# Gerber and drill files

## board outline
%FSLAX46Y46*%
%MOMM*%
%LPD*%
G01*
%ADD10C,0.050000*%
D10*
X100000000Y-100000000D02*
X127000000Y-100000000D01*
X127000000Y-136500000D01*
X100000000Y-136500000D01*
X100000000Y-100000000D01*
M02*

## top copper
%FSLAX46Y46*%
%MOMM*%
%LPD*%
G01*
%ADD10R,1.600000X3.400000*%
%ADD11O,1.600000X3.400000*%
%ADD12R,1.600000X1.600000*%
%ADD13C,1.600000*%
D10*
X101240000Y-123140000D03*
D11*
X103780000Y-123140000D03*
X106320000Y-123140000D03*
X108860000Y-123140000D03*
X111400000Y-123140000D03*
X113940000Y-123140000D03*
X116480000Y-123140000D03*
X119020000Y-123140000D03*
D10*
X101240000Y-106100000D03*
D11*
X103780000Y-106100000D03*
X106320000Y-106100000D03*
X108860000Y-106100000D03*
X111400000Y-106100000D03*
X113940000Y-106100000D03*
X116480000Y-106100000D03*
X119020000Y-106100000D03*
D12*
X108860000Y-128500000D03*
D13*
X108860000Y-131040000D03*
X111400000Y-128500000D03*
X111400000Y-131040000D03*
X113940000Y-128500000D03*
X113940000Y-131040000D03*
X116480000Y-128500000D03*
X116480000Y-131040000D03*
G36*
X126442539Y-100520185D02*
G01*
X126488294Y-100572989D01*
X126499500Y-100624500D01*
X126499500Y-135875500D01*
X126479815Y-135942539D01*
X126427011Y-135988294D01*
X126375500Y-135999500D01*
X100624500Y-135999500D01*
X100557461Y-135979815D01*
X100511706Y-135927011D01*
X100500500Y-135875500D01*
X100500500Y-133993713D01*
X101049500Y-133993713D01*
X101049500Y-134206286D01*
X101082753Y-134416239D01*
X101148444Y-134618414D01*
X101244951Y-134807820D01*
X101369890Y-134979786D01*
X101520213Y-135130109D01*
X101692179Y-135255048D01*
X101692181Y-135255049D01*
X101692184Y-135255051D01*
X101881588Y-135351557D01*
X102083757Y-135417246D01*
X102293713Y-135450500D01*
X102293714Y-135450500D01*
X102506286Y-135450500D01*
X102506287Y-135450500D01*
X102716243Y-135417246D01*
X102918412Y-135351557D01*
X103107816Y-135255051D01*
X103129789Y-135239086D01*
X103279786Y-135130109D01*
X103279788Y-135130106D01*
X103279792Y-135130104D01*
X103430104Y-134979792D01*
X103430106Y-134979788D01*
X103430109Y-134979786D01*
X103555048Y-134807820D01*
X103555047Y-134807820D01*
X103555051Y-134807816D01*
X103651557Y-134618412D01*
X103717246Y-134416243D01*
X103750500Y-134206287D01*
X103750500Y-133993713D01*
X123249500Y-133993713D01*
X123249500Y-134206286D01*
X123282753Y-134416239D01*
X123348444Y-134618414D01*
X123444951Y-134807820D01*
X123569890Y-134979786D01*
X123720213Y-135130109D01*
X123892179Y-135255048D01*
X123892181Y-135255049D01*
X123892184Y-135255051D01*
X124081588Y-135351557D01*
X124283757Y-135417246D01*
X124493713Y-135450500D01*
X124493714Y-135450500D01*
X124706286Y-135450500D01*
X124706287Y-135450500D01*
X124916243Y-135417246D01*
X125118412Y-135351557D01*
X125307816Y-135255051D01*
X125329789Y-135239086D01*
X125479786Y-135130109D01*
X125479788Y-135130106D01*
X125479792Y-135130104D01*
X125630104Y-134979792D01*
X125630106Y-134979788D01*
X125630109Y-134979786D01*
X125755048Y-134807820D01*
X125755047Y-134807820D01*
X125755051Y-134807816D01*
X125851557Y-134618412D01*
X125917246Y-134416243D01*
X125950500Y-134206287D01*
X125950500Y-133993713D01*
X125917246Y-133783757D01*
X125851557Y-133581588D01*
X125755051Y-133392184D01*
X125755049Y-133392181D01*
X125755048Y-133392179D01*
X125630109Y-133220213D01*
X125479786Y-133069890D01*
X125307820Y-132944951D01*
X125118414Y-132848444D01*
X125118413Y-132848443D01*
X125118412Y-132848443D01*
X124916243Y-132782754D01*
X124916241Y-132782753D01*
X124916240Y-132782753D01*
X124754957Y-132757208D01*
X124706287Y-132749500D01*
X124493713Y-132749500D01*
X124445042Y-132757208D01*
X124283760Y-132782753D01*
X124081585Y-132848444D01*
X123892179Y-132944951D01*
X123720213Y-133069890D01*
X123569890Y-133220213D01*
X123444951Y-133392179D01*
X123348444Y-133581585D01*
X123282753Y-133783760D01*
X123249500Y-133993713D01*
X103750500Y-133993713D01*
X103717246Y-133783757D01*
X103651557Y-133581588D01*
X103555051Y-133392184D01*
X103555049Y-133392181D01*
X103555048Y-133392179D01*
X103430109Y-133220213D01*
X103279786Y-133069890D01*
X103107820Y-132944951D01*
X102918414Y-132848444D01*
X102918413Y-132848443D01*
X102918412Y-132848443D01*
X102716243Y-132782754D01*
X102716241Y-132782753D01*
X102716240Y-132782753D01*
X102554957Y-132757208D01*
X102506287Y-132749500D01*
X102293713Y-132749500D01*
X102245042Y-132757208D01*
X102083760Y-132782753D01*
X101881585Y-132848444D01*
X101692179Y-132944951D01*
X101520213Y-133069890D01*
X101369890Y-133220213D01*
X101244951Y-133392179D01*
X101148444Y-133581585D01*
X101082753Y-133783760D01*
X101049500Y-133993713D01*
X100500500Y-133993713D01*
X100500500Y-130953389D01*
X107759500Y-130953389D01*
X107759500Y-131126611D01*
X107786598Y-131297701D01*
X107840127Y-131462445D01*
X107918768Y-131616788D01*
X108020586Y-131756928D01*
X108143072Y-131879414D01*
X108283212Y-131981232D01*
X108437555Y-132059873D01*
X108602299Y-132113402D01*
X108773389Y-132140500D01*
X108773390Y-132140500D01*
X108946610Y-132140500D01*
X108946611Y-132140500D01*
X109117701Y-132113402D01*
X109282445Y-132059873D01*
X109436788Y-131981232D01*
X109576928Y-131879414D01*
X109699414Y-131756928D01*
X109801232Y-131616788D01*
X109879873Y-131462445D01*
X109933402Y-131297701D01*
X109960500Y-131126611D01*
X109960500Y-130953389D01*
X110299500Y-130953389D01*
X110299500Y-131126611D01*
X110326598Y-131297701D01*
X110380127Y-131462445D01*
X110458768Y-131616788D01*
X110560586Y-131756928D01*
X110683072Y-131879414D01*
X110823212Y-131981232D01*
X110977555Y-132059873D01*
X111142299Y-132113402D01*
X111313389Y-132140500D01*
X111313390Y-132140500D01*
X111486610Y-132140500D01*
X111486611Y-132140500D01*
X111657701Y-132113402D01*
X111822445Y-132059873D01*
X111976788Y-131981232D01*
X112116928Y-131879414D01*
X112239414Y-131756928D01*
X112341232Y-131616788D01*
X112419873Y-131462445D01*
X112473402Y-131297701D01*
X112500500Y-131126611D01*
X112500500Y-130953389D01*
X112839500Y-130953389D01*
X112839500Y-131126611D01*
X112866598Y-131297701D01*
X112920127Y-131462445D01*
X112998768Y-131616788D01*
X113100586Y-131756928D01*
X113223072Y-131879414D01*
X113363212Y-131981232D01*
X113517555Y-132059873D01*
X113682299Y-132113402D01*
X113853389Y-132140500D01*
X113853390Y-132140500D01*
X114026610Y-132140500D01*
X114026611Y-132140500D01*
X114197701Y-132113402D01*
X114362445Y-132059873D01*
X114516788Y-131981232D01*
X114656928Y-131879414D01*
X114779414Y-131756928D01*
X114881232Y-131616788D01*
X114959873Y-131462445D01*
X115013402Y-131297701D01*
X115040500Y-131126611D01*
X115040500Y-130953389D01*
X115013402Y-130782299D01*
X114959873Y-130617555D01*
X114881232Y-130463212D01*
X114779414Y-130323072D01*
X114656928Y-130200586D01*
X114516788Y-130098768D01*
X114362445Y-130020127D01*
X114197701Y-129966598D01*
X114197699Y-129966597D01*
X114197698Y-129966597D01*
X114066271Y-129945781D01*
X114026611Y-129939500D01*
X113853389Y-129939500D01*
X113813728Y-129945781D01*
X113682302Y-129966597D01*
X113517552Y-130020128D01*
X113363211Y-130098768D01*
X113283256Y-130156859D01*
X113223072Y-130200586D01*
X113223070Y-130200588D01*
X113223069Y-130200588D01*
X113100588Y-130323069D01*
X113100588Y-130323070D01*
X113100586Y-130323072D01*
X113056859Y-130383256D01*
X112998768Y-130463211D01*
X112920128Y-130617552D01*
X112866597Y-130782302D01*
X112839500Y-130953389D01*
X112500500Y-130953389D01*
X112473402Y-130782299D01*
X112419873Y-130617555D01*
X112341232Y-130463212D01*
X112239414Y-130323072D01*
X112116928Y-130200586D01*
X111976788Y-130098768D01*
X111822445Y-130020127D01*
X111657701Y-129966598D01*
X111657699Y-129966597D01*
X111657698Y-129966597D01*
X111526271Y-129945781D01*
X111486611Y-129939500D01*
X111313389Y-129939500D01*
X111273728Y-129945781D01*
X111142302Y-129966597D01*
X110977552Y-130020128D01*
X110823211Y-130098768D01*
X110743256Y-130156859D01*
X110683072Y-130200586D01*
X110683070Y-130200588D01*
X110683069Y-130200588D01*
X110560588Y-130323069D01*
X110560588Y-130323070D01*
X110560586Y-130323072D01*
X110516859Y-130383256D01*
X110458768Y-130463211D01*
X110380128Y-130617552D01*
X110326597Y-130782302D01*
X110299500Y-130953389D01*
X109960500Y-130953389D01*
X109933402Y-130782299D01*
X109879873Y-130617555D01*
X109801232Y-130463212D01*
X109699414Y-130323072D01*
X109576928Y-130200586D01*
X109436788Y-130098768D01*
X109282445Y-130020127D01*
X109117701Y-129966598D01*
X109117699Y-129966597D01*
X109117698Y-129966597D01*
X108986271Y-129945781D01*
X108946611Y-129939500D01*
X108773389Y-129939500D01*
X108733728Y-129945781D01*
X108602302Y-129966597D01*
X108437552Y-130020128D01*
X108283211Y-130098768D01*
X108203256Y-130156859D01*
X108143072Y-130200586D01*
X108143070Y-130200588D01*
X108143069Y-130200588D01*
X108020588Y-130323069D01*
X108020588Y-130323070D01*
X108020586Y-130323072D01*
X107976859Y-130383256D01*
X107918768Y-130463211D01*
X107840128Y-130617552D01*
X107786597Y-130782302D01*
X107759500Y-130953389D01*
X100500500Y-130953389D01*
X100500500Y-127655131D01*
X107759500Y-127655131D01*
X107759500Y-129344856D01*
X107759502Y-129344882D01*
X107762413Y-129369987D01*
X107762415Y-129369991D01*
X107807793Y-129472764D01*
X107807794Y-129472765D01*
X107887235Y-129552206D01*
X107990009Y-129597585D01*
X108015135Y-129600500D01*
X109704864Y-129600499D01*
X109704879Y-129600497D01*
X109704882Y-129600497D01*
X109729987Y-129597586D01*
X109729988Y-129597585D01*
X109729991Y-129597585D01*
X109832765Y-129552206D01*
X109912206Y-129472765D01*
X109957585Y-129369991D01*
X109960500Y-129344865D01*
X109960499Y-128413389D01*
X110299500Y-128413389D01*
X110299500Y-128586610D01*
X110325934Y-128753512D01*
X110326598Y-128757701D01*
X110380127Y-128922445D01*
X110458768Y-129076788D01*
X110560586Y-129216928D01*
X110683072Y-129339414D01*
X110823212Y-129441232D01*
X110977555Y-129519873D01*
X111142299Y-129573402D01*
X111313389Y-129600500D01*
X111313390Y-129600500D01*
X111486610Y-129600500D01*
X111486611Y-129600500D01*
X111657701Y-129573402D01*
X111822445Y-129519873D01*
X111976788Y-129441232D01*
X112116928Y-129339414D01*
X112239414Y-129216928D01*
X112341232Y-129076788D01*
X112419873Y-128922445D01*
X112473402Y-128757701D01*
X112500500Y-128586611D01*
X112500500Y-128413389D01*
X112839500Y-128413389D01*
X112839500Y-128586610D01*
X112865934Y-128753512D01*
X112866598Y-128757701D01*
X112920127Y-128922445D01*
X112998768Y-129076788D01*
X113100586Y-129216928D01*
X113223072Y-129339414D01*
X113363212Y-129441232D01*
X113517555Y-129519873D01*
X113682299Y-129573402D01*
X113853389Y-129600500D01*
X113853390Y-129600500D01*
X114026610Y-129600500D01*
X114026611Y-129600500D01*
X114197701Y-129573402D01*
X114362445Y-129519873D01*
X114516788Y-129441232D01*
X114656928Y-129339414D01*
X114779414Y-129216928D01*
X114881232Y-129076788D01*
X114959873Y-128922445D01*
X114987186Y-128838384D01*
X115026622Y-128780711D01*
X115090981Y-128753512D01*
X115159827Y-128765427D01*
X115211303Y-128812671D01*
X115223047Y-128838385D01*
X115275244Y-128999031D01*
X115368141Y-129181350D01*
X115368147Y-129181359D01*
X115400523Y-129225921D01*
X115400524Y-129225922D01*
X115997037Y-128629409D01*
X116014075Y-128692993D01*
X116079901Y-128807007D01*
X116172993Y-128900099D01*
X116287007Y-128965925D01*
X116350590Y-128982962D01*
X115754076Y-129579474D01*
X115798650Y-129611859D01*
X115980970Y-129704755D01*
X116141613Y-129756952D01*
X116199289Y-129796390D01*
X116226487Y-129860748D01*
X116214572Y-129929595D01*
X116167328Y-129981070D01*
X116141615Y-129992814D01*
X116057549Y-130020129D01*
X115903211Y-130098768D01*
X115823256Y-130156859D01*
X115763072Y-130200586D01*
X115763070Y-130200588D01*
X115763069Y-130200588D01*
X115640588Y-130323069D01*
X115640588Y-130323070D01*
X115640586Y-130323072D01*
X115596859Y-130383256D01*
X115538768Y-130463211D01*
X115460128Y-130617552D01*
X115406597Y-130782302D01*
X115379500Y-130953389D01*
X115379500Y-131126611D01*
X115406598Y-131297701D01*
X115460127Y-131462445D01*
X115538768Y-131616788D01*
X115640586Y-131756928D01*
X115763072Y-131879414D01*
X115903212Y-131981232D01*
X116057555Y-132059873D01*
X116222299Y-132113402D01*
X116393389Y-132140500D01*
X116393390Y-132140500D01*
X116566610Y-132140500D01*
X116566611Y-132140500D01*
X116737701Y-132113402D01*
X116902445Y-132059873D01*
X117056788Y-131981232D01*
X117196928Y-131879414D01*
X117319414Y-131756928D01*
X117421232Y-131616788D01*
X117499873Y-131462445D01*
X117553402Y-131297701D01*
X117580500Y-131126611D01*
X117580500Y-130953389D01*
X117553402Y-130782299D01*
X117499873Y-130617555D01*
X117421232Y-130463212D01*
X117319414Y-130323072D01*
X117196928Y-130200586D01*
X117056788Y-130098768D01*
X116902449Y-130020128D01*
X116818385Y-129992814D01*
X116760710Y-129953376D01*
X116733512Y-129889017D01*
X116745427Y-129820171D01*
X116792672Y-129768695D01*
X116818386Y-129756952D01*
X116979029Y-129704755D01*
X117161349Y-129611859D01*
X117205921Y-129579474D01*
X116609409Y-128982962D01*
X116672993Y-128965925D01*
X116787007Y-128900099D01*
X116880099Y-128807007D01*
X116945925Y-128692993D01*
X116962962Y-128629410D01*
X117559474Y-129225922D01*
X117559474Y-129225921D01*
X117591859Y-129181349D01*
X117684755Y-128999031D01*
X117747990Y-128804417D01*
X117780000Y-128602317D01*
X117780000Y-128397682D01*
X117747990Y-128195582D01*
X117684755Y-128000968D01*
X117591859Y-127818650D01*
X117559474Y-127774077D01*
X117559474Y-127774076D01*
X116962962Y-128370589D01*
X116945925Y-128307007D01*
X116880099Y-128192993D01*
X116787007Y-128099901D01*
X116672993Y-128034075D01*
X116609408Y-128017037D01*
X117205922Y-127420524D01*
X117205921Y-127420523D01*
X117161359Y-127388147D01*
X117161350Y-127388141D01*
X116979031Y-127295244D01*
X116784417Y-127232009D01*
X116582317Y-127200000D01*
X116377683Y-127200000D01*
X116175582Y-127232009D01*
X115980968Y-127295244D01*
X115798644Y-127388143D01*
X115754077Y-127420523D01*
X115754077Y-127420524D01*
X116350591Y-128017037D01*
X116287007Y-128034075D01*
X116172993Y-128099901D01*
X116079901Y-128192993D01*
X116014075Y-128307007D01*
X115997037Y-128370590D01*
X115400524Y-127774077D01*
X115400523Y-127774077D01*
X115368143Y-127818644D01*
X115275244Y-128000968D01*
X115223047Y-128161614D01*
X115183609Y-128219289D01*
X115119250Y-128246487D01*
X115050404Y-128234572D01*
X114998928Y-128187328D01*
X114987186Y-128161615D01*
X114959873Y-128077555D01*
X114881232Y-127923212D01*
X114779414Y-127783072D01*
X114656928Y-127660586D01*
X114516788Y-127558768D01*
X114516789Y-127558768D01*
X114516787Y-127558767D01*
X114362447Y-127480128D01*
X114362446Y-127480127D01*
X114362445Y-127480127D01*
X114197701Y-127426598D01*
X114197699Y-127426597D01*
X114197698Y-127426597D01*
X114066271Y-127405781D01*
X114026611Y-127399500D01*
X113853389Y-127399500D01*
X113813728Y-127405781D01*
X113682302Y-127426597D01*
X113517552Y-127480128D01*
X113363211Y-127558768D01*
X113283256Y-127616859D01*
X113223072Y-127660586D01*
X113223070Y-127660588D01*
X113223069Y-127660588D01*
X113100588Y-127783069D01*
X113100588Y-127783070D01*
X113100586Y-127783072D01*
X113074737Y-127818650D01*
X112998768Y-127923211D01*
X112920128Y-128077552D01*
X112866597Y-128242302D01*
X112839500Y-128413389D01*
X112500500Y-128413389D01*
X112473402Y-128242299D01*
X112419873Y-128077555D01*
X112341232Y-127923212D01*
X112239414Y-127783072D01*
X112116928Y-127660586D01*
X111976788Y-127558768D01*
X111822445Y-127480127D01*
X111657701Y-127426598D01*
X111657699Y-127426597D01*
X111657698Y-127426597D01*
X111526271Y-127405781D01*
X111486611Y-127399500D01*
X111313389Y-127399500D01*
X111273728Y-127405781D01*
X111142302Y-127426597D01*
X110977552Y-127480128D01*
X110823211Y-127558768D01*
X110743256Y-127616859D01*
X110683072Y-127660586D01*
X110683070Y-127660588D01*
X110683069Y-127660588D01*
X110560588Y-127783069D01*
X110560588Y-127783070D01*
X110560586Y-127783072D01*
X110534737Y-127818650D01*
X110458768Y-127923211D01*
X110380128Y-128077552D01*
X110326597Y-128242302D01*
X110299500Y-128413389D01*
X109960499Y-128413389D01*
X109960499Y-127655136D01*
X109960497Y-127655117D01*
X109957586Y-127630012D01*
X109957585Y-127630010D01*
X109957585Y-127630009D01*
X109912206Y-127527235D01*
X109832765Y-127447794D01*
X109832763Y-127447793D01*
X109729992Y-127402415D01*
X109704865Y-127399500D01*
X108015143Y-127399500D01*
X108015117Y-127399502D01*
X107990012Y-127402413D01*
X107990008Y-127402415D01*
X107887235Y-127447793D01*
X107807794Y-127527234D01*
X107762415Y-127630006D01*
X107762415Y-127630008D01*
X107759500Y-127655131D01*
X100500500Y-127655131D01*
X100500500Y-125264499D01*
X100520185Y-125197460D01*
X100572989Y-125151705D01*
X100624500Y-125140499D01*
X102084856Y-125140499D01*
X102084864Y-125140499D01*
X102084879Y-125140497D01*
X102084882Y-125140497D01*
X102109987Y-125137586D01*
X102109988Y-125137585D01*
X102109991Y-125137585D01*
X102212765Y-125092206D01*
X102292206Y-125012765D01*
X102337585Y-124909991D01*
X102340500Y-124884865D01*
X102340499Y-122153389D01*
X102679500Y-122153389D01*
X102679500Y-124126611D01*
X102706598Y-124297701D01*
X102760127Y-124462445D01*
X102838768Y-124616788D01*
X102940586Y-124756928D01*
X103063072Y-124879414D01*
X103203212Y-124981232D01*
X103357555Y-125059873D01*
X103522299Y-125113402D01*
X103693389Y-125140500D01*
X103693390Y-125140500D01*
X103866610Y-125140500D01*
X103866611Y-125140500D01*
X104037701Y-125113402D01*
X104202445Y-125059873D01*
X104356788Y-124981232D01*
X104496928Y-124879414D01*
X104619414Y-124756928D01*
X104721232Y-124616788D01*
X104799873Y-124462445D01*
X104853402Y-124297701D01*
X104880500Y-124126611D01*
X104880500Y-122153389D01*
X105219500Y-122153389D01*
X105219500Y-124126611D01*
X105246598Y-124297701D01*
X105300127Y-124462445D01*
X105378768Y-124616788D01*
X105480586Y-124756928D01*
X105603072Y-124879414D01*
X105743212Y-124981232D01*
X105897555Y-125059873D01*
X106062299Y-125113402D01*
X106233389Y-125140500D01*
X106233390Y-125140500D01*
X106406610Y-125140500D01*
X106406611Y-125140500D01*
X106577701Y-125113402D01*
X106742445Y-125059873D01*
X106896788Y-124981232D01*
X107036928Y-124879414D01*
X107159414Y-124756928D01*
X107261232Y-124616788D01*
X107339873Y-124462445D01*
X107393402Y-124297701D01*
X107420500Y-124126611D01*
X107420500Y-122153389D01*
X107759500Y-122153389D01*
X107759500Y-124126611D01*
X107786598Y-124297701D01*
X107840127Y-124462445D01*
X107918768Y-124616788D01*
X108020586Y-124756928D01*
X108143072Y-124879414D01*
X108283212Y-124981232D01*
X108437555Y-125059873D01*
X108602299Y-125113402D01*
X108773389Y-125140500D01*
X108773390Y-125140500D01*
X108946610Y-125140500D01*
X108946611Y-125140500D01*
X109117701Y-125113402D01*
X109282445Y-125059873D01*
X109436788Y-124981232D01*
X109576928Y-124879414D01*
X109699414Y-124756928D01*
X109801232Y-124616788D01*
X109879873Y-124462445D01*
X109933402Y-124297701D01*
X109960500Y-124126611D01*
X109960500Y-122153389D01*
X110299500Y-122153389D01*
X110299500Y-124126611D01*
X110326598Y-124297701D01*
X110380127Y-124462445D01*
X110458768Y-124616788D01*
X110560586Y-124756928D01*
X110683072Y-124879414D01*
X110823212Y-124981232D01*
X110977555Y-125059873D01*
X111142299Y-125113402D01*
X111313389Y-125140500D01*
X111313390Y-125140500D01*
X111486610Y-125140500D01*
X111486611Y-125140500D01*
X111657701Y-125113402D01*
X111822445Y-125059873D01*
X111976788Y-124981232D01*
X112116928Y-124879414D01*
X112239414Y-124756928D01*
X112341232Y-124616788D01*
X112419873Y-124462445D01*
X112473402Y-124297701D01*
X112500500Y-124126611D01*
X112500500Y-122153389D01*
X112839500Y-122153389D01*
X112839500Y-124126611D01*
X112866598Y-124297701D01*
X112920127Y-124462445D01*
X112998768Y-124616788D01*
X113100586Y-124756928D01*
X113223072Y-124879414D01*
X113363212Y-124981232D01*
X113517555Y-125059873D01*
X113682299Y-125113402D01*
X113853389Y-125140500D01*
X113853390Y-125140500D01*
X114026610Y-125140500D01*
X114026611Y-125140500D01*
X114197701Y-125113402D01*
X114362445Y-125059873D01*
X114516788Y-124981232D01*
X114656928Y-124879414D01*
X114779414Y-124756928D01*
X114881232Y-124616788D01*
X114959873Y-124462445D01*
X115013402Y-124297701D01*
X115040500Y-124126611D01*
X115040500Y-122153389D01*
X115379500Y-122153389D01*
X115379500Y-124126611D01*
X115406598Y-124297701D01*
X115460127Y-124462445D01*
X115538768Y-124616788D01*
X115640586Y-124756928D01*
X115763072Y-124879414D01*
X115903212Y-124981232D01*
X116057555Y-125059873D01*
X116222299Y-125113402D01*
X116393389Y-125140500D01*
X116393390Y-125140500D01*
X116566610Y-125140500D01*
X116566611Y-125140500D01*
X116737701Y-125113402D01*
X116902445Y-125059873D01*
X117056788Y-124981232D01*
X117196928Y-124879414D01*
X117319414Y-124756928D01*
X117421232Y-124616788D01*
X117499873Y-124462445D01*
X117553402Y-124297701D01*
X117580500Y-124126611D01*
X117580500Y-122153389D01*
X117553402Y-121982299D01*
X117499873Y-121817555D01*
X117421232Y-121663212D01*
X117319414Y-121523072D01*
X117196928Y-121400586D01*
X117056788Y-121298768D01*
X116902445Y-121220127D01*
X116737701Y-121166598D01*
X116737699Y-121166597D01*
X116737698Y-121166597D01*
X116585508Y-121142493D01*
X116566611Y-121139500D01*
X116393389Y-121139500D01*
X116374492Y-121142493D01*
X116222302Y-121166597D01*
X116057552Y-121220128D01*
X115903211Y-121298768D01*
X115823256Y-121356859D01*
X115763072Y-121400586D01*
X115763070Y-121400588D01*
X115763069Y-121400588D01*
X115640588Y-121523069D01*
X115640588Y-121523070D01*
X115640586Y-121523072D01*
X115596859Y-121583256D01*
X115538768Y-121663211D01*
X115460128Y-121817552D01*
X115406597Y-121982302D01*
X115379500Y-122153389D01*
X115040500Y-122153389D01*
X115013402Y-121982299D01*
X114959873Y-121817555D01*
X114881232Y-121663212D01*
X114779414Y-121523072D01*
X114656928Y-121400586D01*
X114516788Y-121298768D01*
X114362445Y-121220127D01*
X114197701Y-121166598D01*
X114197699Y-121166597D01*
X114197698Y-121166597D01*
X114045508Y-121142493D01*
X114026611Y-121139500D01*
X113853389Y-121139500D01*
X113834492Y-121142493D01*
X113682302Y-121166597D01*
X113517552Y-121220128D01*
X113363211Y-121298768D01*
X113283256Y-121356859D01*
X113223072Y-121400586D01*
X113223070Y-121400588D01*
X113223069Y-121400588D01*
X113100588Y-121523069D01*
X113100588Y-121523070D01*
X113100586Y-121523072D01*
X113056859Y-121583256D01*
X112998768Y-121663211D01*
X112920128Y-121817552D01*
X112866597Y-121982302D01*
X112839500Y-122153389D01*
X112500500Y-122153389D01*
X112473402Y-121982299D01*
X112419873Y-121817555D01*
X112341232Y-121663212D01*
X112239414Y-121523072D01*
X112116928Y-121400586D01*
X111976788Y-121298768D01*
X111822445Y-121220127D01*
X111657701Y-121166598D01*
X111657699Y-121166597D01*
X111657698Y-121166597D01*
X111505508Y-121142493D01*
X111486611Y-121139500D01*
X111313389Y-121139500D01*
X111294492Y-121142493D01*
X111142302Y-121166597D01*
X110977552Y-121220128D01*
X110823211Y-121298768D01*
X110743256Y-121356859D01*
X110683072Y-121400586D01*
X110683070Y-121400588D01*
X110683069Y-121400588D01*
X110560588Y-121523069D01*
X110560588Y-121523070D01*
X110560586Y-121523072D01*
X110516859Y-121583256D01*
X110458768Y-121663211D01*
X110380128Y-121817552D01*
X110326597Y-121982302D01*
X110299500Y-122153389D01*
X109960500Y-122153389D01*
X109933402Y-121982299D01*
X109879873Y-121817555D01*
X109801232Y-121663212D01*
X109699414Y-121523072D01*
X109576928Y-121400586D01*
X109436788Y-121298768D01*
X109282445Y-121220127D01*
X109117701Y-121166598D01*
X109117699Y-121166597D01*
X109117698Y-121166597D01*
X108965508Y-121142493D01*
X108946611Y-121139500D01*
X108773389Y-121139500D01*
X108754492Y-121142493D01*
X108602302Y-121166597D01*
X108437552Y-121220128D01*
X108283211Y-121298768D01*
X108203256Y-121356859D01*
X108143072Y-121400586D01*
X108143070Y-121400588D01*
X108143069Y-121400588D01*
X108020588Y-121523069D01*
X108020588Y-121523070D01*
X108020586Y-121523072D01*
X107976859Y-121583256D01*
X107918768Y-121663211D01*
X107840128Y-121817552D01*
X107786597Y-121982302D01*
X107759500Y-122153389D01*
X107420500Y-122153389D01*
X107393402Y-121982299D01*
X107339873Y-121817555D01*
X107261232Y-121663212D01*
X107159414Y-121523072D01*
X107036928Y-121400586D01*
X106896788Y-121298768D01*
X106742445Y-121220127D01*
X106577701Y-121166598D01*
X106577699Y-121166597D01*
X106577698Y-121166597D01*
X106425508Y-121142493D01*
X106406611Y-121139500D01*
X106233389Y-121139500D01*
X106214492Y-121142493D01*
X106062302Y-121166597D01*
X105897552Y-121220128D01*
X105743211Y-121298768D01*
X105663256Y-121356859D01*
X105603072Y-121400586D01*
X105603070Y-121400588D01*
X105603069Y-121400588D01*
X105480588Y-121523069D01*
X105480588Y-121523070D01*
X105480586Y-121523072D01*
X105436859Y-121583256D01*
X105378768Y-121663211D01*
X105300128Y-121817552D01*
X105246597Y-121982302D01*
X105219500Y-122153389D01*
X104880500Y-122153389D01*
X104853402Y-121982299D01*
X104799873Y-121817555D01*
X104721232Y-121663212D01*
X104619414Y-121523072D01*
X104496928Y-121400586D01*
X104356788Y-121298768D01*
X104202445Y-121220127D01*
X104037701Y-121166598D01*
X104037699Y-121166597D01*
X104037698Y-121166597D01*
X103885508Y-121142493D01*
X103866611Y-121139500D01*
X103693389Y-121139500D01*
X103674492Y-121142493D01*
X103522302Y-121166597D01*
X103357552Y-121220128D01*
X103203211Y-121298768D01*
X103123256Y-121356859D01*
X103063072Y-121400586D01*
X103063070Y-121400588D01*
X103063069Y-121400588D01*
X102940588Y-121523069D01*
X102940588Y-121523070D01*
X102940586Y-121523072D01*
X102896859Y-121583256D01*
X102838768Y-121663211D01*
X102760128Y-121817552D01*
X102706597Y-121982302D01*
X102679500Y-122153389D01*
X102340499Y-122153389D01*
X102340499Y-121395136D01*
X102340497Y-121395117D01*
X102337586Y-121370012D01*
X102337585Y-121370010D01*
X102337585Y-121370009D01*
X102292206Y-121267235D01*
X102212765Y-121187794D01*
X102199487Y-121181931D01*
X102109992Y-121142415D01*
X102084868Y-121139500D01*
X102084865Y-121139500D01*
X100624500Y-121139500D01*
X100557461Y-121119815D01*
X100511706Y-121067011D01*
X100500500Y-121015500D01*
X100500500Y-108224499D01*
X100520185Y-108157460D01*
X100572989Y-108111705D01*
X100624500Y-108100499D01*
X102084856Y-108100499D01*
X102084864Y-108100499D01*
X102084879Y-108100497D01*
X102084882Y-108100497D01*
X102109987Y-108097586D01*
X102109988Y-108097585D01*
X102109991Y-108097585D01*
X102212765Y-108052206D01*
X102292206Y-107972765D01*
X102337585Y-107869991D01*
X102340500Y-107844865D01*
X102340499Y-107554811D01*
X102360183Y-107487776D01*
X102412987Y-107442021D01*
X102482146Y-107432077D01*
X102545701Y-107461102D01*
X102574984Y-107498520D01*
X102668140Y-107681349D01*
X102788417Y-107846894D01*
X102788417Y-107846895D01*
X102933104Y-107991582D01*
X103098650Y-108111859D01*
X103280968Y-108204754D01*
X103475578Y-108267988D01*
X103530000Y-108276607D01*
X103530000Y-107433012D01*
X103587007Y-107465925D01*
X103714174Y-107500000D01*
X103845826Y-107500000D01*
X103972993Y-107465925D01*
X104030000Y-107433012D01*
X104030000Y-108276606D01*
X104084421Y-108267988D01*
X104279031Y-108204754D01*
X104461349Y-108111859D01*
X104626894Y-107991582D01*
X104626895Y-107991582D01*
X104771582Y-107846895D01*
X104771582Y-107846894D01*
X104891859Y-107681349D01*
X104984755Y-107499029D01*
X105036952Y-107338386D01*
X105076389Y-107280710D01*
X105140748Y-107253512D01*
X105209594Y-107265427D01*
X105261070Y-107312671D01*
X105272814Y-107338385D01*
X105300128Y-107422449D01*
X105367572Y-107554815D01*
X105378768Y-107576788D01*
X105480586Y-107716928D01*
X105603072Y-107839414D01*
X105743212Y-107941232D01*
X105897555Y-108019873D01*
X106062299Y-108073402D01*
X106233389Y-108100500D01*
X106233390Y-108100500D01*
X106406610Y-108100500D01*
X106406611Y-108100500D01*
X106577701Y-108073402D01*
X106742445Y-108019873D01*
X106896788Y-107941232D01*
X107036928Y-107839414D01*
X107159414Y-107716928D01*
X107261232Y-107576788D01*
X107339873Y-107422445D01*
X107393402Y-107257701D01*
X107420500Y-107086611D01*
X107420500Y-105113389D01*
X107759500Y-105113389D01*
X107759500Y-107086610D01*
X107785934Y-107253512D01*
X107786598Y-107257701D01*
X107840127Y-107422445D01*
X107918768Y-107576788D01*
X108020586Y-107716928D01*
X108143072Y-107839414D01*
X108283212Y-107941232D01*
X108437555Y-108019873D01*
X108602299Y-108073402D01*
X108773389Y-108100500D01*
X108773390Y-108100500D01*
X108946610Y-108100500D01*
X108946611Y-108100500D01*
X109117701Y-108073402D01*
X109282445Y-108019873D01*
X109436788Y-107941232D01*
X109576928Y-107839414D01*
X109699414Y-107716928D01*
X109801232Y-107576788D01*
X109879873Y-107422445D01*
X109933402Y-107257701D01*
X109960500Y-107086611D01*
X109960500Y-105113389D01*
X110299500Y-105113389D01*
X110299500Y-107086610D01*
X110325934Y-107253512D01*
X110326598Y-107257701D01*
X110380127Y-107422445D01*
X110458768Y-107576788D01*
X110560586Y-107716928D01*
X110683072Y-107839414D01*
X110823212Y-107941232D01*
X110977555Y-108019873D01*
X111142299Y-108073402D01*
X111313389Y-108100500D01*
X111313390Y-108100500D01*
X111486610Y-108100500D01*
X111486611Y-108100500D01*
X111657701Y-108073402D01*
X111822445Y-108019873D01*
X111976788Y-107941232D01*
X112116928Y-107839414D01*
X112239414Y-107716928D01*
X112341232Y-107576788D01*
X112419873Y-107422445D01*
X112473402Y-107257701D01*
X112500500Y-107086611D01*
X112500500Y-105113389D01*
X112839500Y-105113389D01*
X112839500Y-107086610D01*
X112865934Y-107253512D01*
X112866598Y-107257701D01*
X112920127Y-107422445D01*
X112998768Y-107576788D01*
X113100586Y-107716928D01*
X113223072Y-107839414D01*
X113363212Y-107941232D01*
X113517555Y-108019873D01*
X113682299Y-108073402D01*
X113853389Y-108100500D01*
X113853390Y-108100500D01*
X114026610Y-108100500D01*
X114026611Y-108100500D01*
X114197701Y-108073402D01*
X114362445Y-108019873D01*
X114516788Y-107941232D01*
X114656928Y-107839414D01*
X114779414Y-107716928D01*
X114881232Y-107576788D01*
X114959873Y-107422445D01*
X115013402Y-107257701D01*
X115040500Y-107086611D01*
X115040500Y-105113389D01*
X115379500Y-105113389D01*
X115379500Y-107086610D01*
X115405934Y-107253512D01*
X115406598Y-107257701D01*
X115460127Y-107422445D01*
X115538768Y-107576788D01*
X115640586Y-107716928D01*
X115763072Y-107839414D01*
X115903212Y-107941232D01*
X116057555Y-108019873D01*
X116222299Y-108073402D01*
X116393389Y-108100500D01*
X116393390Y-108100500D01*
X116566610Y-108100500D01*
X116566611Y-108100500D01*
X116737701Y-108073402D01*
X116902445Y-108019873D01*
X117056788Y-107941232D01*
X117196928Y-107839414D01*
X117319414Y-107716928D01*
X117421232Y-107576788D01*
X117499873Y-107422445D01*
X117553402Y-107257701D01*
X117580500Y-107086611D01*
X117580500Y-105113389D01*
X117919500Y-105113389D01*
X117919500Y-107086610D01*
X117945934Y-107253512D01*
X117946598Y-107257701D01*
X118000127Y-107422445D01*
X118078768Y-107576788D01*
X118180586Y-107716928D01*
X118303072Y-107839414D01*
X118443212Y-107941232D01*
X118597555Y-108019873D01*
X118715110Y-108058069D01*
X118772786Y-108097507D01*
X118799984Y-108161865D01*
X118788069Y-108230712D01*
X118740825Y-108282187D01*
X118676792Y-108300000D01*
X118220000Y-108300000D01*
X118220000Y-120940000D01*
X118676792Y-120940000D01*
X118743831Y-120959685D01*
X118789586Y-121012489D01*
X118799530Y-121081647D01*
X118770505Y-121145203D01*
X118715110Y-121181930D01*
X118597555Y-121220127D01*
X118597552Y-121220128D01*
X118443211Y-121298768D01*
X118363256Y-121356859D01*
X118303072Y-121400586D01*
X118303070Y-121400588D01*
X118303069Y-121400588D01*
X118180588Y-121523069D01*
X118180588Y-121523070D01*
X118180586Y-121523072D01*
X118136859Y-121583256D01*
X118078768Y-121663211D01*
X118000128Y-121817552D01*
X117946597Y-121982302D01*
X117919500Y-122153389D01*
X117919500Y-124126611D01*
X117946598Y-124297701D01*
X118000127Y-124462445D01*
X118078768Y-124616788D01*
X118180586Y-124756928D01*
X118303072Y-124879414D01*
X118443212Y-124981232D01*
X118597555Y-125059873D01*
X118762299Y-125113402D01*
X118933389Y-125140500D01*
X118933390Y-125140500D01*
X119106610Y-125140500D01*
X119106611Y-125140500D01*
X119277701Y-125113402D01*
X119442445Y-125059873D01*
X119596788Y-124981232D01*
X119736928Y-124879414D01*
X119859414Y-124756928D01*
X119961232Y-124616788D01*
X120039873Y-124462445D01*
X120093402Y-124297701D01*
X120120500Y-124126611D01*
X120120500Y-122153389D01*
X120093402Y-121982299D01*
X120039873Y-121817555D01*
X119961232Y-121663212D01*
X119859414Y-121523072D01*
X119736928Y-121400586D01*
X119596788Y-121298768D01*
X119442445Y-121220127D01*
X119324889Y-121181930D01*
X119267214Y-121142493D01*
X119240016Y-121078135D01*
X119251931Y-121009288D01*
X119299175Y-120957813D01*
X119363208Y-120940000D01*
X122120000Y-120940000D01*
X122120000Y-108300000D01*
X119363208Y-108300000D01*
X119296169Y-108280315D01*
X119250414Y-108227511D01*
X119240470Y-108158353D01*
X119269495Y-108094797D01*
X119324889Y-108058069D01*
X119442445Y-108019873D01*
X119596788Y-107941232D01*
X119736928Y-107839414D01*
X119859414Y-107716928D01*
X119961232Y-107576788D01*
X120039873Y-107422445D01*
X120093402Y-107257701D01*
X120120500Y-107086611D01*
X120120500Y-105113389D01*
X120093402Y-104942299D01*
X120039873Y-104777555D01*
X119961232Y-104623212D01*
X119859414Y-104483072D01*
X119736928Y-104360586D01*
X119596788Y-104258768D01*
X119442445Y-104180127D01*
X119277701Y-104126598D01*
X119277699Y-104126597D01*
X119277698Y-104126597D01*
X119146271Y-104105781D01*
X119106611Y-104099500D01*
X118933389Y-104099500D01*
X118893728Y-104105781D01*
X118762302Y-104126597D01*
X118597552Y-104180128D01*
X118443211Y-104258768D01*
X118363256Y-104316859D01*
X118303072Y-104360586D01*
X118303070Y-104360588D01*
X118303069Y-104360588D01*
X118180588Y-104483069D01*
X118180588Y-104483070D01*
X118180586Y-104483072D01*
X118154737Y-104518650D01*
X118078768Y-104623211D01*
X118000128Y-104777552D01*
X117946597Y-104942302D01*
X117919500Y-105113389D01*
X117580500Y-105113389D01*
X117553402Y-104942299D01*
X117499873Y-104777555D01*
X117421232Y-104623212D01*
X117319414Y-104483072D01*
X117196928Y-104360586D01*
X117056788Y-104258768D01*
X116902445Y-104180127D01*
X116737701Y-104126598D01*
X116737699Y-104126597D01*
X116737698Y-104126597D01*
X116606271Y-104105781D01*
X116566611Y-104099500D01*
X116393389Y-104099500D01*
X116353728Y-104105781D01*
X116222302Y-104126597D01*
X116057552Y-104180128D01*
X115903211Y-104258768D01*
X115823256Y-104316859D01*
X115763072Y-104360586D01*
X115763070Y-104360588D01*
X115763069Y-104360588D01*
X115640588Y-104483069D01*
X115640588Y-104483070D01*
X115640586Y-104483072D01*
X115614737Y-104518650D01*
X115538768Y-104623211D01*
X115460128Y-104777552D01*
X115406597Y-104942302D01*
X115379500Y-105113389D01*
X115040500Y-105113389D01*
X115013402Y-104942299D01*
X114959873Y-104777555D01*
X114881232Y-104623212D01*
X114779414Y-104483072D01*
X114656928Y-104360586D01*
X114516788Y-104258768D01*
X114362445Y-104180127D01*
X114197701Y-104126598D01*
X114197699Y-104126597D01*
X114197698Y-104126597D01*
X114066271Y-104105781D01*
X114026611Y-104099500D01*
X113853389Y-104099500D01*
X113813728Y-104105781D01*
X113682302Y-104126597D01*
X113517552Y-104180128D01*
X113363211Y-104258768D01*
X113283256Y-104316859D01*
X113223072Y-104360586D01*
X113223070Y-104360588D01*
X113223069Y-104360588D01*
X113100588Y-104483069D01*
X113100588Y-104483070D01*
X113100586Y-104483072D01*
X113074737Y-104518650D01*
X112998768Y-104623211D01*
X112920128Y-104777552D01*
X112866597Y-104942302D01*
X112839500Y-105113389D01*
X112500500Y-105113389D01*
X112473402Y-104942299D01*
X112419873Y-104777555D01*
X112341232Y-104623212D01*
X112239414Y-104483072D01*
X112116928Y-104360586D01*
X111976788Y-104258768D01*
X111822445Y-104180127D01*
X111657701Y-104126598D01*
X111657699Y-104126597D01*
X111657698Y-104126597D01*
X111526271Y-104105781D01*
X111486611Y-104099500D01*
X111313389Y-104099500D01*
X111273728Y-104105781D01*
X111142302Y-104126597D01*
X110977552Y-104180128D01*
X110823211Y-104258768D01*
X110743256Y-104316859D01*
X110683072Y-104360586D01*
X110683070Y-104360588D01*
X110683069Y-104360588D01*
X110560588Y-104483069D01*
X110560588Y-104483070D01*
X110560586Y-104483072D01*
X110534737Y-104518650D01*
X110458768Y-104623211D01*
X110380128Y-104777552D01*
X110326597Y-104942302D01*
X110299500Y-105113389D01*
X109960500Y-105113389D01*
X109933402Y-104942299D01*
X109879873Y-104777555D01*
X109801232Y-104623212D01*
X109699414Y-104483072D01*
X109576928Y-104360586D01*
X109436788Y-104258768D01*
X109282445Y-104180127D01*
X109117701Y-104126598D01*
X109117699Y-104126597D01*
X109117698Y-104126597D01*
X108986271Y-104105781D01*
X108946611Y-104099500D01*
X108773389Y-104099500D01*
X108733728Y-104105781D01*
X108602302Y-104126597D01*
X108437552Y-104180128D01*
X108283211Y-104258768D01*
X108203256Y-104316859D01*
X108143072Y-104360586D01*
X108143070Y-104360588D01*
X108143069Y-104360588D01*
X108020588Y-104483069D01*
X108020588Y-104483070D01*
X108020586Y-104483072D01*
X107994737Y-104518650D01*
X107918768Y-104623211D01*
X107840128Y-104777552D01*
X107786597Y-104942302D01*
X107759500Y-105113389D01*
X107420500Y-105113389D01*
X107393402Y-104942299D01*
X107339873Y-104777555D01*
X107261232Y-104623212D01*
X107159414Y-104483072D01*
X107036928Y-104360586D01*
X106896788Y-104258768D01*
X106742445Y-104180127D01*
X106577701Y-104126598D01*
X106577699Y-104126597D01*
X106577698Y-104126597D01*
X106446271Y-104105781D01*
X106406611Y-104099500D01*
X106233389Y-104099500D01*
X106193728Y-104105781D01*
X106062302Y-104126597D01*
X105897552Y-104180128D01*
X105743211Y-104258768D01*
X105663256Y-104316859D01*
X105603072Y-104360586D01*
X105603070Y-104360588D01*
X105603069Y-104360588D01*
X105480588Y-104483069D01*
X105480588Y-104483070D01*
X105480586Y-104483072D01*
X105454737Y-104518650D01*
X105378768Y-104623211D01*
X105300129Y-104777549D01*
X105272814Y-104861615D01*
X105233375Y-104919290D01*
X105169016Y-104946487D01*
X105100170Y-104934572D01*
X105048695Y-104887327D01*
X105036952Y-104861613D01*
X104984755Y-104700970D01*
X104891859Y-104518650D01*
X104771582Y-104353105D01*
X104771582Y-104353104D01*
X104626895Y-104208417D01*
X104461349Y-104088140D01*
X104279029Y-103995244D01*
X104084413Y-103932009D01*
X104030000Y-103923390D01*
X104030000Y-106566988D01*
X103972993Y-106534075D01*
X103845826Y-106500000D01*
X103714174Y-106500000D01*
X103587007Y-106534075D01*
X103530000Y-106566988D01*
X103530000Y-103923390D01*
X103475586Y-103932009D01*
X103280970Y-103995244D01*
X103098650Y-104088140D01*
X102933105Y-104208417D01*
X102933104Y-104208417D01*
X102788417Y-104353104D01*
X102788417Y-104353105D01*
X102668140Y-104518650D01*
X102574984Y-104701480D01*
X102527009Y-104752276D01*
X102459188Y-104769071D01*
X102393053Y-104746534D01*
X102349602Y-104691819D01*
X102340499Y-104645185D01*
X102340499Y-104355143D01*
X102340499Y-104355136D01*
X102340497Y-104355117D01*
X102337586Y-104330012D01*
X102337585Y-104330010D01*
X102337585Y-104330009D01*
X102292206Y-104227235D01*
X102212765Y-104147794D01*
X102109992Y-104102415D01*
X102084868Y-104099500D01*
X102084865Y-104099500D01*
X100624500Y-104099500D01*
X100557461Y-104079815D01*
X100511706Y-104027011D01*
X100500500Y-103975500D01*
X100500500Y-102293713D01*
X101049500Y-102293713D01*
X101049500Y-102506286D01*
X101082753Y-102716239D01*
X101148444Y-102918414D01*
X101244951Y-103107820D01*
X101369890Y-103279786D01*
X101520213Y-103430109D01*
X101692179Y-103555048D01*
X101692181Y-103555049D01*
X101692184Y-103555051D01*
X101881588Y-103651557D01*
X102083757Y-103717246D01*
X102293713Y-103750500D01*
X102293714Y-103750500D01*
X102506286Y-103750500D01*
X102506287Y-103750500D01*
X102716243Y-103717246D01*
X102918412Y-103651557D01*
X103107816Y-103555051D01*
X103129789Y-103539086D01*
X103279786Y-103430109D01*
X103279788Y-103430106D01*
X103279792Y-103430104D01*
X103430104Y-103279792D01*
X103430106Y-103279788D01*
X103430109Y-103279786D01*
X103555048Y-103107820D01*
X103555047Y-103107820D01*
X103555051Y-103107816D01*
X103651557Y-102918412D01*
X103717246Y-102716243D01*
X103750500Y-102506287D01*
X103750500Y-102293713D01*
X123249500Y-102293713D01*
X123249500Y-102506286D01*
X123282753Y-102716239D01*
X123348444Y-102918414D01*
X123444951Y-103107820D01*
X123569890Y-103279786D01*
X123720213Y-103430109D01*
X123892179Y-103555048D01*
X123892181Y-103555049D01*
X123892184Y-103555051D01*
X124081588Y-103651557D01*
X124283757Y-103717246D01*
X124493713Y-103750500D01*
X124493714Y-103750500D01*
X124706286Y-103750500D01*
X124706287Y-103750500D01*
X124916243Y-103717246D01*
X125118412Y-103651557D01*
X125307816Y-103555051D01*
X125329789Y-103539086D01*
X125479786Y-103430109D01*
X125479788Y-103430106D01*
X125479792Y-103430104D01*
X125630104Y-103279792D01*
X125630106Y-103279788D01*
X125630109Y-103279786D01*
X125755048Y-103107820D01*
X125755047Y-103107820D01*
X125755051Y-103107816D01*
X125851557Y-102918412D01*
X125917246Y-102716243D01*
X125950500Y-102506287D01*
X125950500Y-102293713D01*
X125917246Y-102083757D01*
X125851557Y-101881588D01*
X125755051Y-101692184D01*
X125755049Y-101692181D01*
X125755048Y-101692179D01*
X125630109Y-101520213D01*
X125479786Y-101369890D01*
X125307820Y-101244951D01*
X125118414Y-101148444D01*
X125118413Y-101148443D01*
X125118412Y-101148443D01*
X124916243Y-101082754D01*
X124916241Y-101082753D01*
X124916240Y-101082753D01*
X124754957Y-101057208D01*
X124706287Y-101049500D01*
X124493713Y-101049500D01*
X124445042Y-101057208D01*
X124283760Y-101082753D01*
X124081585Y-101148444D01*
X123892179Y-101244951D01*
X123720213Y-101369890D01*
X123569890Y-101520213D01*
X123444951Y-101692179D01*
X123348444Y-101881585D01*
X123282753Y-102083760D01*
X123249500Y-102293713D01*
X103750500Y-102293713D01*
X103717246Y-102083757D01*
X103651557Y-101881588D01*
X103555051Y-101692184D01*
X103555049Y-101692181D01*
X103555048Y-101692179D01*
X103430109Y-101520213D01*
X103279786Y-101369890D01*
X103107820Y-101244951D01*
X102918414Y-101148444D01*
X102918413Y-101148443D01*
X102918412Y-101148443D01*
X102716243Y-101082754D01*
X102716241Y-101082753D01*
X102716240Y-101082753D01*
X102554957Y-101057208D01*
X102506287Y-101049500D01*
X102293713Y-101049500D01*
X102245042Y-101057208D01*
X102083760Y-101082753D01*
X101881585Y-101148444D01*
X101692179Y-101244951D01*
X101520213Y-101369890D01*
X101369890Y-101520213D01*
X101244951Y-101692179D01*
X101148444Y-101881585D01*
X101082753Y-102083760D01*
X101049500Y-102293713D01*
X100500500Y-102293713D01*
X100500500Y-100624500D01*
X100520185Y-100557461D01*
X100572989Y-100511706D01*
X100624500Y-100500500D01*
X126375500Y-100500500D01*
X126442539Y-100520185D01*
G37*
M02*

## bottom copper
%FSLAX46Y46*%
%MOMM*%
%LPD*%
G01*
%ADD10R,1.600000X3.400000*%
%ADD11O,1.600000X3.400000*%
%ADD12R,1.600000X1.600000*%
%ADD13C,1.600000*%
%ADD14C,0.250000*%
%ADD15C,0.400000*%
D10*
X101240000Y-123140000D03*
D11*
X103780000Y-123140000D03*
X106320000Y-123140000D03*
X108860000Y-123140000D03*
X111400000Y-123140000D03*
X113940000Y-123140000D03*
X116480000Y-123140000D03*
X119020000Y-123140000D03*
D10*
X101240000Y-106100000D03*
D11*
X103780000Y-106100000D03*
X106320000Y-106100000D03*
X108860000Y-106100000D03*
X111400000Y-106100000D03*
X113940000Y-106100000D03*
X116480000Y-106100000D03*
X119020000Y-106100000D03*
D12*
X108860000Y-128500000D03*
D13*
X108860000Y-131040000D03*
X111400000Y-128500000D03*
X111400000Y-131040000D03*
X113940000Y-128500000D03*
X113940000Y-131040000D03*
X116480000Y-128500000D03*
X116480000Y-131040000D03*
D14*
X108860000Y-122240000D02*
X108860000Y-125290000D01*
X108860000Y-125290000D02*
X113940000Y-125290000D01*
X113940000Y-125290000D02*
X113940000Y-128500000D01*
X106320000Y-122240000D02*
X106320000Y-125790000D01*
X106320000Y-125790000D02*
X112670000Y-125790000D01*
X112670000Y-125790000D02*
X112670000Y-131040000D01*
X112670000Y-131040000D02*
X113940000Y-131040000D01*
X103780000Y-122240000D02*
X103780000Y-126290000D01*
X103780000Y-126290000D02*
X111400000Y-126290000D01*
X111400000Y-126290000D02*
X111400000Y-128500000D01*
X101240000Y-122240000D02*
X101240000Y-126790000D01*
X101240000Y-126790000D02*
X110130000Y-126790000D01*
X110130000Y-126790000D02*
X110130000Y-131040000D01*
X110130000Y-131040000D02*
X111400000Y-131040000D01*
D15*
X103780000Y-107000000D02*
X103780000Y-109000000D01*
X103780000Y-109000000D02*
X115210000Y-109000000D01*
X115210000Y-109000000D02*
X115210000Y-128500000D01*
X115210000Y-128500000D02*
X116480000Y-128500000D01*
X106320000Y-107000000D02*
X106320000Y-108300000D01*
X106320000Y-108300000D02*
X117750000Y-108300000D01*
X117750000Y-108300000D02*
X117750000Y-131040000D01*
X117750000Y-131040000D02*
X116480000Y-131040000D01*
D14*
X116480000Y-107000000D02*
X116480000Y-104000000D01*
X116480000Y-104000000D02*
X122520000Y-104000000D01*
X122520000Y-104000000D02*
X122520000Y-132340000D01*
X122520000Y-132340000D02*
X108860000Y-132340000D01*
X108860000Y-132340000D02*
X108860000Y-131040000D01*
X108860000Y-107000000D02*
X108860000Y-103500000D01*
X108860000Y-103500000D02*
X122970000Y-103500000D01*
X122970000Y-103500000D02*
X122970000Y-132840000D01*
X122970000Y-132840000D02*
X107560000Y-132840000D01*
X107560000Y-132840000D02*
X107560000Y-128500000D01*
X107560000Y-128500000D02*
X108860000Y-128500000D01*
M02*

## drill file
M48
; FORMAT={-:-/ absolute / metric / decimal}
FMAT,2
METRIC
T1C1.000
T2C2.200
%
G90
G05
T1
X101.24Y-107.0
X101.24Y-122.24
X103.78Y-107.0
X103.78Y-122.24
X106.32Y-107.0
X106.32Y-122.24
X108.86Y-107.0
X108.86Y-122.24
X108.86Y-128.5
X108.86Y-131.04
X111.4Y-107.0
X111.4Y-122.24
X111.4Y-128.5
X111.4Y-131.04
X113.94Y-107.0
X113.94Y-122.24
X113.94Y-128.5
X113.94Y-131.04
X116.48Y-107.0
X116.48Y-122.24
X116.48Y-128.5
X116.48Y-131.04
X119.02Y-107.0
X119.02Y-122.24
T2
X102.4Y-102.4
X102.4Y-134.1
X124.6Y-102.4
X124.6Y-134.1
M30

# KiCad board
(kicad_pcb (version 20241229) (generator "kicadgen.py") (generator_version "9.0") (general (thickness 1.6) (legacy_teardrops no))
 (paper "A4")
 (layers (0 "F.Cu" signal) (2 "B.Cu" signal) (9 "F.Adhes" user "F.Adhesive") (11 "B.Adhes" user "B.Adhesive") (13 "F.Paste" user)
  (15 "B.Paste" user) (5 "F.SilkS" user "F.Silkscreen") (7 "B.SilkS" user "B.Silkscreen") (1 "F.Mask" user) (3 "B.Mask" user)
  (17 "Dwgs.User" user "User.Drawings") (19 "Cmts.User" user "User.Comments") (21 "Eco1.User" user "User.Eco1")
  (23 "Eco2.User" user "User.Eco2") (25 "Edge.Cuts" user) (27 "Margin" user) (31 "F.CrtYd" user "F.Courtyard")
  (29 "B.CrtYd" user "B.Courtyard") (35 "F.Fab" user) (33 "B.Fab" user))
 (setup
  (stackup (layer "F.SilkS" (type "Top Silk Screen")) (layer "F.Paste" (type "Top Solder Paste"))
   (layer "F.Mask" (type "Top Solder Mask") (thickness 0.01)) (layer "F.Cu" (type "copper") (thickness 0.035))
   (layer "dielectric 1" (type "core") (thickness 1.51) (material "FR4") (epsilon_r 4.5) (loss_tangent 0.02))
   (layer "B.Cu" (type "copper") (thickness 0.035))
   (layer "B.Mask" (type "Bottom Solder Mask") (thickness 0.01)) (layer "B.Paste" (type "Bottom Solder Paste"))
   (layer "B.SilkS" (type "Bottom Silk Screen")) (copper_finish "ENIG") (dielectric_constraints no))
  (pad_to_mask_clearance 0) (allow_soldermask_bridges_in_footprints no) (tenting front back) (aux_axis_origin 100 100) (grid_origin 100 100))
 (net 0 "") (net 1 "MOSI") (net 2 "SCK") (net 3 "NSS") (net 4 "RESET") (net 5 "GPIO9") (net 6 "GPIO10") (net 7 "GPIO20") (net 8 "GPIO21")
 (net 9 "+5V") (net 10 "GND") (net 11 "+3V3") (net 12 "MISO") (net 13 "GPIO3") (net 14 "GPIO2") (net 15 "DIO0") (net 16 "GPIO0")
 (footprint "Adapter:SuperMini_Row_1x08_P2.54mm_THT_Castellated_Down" (layer "F.Cu") (at 101.24 122.24)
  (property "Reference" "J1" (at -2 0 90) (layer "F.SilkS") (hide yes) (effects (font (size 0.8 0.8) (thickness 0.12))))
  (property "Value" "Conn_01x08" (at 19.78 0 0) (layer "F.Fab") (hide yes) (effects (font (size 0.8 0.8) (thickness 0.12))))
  (pad "1" thru_hole rect (at 0 0) (size 1.6 3.4) (drill 1 (offset 0 0.9)) (layers "*.Cu" "*.Mask") (remove_unused_layers no) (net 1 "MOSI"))
  (pad "2" thru_hole oval (at 2.54 0) (size 1.6 3.4) (drill 1 (offset 0 0.9)) (layers "*.Cu" "*.Mask") (remove_unused_layers no)
   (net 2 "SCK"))
  (pad "3" thru_hole oval (at 5.08 0) (size 1.6 3.4) (drill 1 (offset 0 0.9)) (layers "*.Cu" "*.Mask") (remove_unused_layers no)
   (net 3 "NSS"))
  (pad "4" thru_hole oval (at 7.62 0) (size 1.6 3.4) (drill 1 (offset 0 0.9)) (layers "*.Cu" "*.Mask") (remove_unused_layers no)
   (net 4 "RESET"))
  (pad "5" thru_hole oval (at 10.16 0) (size 1.6 3.4) (drill 1 (offset 0 0.9)) (layers "*.Cu" "*.Mask") (remove_unused_layers no)
   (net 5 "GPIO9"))
  (pad "6" thru_hole oval (at 12.7 0) (size 1.6 3.4) (drill 1 (offset 0 0.9)) (layers "*.Cu" "*.Mask") (remove_unused_layers no)
   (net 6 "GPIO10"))
  (pad "7" thru_hole oval (at 15.24 0) (size 1.6 3.4) (drill 1 (offset 0 0.9)) (layers "*.Cu" "*.Mask") (remove_unused_layers no)
   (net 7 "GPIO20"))
  (pad "8" thru_hole oval (at 17.78 0) (size 1.6 3.4) (drill 1 (offset 0 0.9)) (layers "*.Cu" "*.Mask") (remove_unused_layers no)
   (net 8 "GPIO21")))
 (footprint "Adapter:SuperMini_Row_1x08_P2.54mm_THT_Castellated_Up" (layer "F.Cu") (at 101.24 107)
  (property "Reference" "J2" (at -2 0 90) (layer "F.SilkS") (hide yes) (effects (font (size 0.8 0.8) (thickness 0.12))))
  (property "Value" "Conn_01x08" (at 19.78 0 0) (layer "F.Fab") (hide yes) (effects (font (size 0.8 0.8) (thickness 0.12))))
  (pad "1" thru_hole rect (at 0 0) (size 1.6 3.4) (drill 1 (offset 0 -0.9)) (layers "*.Cu" "*.Mask") (remove_unused_layers no) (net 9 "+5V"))
  (pad "2" thru_hole oval (at 2.54 0) (size 1.6 3.4) (drill 1 (offset 0 -0.9)) (layers "*.Cu" "*.Mask") (remove_unused_layers no)
   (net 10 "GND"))
  (pad "3" thru_hole oval (at 5.08 0) (size 1.6 3.4) (drill 1 (offset 0 -0.9)) (layers "*.Cu" "*.Mask") (remove_unused_layers no)
   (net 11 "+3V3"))
  (pad "4" thru_hole oval (at 7.62 0) (size 1.6 3.4) (drill 1 (offset 0 -0.9)) (layers "*.Cu" "*.Mask") (remove_unused_layers no)
   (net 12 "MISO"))
  (pad "5" thru_hole oval (at 10.16 0) (size 1.6 3.4) (drill 1 (offset 0 -0.9)) (layers "*.Cu" "*.Mask") (remove_unused_layers no)
   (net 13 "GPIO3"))
  (pad "6" thru_hole oval (at 12.7 0) (size 1.6 3.4) (drill 1 (offset 0 -0.9)) (layers "*.Cu" "*.Mask") (remove_unused_layers no)
   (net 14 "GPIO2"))
  (pad "7" thru_hole oval (at 15.24 0) (size 1.6 3.4) (drill 1 (offset 0 -0.9)) (layers "*.Cu" "*.Mask") (remove_unused_layers no)
   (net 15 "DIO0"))
  (pad "8" thru_hole oval (at 17.78 0) (size 1.6 3.4) (drill 1 (offset 0 -0.9)) (layers "*.Cu" "*.Mask") (remove_unused_layers no)
   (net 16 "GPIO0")))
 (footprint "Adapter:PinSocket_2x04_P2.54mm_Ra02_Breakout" (layer "F.Cu") (at 108.86 128.5)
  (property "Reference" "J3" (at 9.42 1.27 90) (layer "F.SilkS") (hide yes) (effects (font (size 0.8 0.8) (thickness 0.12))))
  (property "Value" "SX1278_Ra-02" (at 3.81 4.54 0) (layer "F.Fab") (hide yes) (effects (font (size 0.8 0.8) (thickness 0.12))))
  (pad "1" thru_hole rect (at 0 0) (size 1.6 1.6) (drill 1) (layers "*.Cu" "*.Mask") (remove_unused_layers no) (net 12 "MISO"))
  (pad "2" thru_hole circle (at 0 2.54) (size 1.6 1.6) (drill 1) (layers "*.Cu" "*.Mask") (remove_unused_layers no) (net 15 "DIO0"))
  (pad "3" thru_hole circle (at 2.54 0) (size 1.6 1.6) (drill 1) (layers "*.Cu" "*.Mask") (remove_unused_layers no) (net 2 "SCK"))
  (pad "4" thru_hole circle (at 2.54 2.54) (size 1.6 1.6) (drill 1) (layers "*.Cu" "*.Mask") (remove_unused_layers no) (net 1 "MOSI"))
  (pad "5" thru_hole circle (at 5.08 0) (size 1.6 1.6) (drill 1) (layers "*.Cu" "*.Mask") (remove_unused_layers no) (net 4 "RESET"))
  (pad "6" thru_hole circle (at 5.08 2.54) (size 1.6 1.6) (drill 1) (layers "*.Cu" "*.Mask") (remove_unused_layers no) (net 3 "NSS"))
  (pad "7" thru_hole circle (at 7.62 0) (size 1.6 1.6) (drill 1) (layers "*.Cu" "*.Mask") (remove_unused_layers no) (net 10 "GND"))
  (pad "8" thru_hole circle (at 7.62 2.54) (size 1.6 1.6) (drill 1) (layers "*.Cu" "*.Mask") (remove_unused_layers no) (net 11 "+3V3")))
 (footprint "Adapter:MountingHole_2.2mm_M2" (layer "F.Cu") (at 102.4 102.4)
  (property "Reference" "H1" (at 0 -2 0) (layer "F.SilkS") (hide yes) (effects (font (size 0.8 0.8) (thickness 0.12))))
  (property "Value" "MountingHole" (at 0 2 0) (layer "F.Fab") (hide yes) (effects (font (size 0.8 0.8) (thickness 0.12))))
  (pad "1" np_thru_hole circle (at 0 0) (size 2.2 2.2) (drill 2.2) (layers "*.Cu" "*.Mask")))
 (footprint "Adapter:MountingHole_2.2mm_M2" (layer "F.Cu") (at 124.6 102.4)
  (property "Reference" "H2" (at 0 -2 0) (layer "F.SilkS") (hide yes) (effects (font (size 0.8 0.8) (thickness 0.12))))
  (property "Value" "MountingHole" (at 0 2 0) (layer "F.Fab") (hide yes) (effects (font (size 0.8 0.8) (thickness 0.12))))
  (pad "1" np_thru_hole circle (at 0 0) (size 2.2 2.2) (drill 2.2) (layers "*.Cu" "*.Mask")))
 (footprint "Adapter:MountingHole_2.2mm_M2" (layer "F.Cu") (at 102.4 134.1)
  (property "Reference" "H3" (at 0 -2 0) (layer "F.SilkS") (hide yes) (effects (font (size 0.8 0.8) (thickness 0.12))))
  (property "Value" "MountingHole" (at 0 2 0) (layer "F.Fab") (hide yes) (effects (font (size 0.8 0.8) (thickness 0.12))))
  (pad "1" np_thru_hole circle (at 0 0) (size 2.2 2.2) (drill 2.2) (layers "*.Cu" "*.Mask")))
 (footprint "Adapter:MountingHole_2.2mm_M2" (layer "F.Cu") (at 124.6 134.1)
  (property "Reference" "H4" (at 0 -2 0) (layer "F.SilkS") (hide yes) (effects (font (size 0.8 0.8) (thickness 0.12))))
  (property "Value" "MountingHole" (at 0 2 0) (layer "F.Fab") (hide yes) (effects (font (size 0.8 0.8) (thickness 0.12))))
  (pad "1" np_thru_hole circle (at 0 0) (size 2.2 2.2) (drill 2.2) (layers "*.Cu" "*.Mask")))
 (gr_rect (start 100 100) (end 127 136.5) (stroke (width 0.05) (type solid)) (fill no) (layer "Edge.Cuts"))
 (segment (start 108.86 122.24) (end 108.86 125.29) (width 0.25) (layer "B.Cu") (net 4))
 (segment (start 108.86 125.29) (end 113.94 125.29) (width 0.25) (layer "B.Cu") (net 4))
 (segment (start 113.94 125.29) (end 113.94 128.5) (width 0.25) (layer "B.Cu") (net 4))
 (segment (start 106.32 122.24) (end 106.32 125.79) (width 0.25) (layer "B.Cu") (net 3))
 (segment (start 106.32 125.79) (end 112.67 125.79) (width 0.25) (layer "B.Cu") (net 3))
 (segment (start 112.67 125.79) (end 112.67 131.04) (width 0.25) (layer "B.Cu") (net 3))
 (segment (start 112.67 131.04) (end 113.94 131.04) (width 0.25) (layer "B.Cu") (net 3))
 (segment (start 103.78 122.24) (end 103.78 126.29) (width 0.25) (layer "B.Cu") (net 2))
 (segment (start 103.78 126.29) (end 111.4 126.29) (width 0.25) (layer "B.Cu") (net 2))
 (segment (start 111.4 126.29) (end 111.4 128.5) (width 0.25) (layer "B.Cu") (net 2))
 (segment (start 101.24 122.24) (end 101.24 126.79) (width 0.25) (layer "B.Cu") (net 1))
 (segment (start 101.24 126.79) (end 110.13 126.79) (width 0.25) (layer "B.Cu") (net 1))
 (segment (start 110.13 126.79) (end 110.13 131.04) (width 0.25) (layer "B.Cu") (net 1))
 (segment (start 110.13 131.04) (end 111.4 131.04) (width 0.25) (layer "B.Cu") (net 1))
 (segment (start 103.78 107) (end 103.78 109) (width 0.4) (layer "B.Cu") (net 10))
 (segment (start 103.78 109) (end 115.21 109) (width 0.4) (layer "B.Cu") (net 10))
 (segment (start 115.21 109) (end 115.21 128.5) (width 0.4) (layer "B.Cu") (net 10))
 (segment (start 115.21 128.5) (end 116.48 128.5) (width 0.4) (layer "B.Cu") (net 10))
 (segment (start 106.32 107) (end 106.32 108.3) (width 0.4) (layer "B.Cu") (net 11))
 (segment (start 106.32 108.3) (end 117.75 108.3) (width 0.4) (layer "B.Cu") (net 11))
 (segment (start 117.75 108.3) (end 117.75 131.04) (width 0.4) (layer "B.Cu") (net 11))
 (segment (start 117.75 131.04) (end 116.48 131.04) (width 0.4) (layer "B.Cu") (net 11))
 (segment (start 116.48 107) (end 116.48 104) (width 0.25) (layer "B.Cu") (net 15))
 (segment (start 116.48 104) (end 122.52 104) (width 0.25) (layer "B.Cu") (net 15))
 (segment (start 122.52 104) (end 122.52 132.34) (width 0.25) (layer "B.Cu") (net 15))
 (segment (start 122.52 132.34) (end 108.86 132.34) (width 0.25) (layer "B.Cu") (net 15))
 (segment (start 108.86 132.34) (end 108.86 131.04) (width 0.25) (layer "B.Cu") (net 15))
 (segment (start 108.86 107) (end 108.86 103.5) (width 0.25) (layer "B.Cu") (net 12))
 (segment (start 108.86 103.5) (end 122.97 103.5) (width 0.25) (layer "B.Cu") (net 12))
 (segment (start 122.97 103.5) (end 122.97 132.84) (width 0.25) (layer "B.Cu") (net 12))
 (segment (start 122.97 132.84) (end 107.56 132.84) (width 0.25) (layer "B.Cu") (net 12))
 (segment (start 107.56 132.84) (end 107.56 128.5) (width 0.25) (layer "B.Cu") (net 12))
 (segment (start 107.56 128.5) (end 108.86 128.5) (width 0.25) (layer "B.Cu") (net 12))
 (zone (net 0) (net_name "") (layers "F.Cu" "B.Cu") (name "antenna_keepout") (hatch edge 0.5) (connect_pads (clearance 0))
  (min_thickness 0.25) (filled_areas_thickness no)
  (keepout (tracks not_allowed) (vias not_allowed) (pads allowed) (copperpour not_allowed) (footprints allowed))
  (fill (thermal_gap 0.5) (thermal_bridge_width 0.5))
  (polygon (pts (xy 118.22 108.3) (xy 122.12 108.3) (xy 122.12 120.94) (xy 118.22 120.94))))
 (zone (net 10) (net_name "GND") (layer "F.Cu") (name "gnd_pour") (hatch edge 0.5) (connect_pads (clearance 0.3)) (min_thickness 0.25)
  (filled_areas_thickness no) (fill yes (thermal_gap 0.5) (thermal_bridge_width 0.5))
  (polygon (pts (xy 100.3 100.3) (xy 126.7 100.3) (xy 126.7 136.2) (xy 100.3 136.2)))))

